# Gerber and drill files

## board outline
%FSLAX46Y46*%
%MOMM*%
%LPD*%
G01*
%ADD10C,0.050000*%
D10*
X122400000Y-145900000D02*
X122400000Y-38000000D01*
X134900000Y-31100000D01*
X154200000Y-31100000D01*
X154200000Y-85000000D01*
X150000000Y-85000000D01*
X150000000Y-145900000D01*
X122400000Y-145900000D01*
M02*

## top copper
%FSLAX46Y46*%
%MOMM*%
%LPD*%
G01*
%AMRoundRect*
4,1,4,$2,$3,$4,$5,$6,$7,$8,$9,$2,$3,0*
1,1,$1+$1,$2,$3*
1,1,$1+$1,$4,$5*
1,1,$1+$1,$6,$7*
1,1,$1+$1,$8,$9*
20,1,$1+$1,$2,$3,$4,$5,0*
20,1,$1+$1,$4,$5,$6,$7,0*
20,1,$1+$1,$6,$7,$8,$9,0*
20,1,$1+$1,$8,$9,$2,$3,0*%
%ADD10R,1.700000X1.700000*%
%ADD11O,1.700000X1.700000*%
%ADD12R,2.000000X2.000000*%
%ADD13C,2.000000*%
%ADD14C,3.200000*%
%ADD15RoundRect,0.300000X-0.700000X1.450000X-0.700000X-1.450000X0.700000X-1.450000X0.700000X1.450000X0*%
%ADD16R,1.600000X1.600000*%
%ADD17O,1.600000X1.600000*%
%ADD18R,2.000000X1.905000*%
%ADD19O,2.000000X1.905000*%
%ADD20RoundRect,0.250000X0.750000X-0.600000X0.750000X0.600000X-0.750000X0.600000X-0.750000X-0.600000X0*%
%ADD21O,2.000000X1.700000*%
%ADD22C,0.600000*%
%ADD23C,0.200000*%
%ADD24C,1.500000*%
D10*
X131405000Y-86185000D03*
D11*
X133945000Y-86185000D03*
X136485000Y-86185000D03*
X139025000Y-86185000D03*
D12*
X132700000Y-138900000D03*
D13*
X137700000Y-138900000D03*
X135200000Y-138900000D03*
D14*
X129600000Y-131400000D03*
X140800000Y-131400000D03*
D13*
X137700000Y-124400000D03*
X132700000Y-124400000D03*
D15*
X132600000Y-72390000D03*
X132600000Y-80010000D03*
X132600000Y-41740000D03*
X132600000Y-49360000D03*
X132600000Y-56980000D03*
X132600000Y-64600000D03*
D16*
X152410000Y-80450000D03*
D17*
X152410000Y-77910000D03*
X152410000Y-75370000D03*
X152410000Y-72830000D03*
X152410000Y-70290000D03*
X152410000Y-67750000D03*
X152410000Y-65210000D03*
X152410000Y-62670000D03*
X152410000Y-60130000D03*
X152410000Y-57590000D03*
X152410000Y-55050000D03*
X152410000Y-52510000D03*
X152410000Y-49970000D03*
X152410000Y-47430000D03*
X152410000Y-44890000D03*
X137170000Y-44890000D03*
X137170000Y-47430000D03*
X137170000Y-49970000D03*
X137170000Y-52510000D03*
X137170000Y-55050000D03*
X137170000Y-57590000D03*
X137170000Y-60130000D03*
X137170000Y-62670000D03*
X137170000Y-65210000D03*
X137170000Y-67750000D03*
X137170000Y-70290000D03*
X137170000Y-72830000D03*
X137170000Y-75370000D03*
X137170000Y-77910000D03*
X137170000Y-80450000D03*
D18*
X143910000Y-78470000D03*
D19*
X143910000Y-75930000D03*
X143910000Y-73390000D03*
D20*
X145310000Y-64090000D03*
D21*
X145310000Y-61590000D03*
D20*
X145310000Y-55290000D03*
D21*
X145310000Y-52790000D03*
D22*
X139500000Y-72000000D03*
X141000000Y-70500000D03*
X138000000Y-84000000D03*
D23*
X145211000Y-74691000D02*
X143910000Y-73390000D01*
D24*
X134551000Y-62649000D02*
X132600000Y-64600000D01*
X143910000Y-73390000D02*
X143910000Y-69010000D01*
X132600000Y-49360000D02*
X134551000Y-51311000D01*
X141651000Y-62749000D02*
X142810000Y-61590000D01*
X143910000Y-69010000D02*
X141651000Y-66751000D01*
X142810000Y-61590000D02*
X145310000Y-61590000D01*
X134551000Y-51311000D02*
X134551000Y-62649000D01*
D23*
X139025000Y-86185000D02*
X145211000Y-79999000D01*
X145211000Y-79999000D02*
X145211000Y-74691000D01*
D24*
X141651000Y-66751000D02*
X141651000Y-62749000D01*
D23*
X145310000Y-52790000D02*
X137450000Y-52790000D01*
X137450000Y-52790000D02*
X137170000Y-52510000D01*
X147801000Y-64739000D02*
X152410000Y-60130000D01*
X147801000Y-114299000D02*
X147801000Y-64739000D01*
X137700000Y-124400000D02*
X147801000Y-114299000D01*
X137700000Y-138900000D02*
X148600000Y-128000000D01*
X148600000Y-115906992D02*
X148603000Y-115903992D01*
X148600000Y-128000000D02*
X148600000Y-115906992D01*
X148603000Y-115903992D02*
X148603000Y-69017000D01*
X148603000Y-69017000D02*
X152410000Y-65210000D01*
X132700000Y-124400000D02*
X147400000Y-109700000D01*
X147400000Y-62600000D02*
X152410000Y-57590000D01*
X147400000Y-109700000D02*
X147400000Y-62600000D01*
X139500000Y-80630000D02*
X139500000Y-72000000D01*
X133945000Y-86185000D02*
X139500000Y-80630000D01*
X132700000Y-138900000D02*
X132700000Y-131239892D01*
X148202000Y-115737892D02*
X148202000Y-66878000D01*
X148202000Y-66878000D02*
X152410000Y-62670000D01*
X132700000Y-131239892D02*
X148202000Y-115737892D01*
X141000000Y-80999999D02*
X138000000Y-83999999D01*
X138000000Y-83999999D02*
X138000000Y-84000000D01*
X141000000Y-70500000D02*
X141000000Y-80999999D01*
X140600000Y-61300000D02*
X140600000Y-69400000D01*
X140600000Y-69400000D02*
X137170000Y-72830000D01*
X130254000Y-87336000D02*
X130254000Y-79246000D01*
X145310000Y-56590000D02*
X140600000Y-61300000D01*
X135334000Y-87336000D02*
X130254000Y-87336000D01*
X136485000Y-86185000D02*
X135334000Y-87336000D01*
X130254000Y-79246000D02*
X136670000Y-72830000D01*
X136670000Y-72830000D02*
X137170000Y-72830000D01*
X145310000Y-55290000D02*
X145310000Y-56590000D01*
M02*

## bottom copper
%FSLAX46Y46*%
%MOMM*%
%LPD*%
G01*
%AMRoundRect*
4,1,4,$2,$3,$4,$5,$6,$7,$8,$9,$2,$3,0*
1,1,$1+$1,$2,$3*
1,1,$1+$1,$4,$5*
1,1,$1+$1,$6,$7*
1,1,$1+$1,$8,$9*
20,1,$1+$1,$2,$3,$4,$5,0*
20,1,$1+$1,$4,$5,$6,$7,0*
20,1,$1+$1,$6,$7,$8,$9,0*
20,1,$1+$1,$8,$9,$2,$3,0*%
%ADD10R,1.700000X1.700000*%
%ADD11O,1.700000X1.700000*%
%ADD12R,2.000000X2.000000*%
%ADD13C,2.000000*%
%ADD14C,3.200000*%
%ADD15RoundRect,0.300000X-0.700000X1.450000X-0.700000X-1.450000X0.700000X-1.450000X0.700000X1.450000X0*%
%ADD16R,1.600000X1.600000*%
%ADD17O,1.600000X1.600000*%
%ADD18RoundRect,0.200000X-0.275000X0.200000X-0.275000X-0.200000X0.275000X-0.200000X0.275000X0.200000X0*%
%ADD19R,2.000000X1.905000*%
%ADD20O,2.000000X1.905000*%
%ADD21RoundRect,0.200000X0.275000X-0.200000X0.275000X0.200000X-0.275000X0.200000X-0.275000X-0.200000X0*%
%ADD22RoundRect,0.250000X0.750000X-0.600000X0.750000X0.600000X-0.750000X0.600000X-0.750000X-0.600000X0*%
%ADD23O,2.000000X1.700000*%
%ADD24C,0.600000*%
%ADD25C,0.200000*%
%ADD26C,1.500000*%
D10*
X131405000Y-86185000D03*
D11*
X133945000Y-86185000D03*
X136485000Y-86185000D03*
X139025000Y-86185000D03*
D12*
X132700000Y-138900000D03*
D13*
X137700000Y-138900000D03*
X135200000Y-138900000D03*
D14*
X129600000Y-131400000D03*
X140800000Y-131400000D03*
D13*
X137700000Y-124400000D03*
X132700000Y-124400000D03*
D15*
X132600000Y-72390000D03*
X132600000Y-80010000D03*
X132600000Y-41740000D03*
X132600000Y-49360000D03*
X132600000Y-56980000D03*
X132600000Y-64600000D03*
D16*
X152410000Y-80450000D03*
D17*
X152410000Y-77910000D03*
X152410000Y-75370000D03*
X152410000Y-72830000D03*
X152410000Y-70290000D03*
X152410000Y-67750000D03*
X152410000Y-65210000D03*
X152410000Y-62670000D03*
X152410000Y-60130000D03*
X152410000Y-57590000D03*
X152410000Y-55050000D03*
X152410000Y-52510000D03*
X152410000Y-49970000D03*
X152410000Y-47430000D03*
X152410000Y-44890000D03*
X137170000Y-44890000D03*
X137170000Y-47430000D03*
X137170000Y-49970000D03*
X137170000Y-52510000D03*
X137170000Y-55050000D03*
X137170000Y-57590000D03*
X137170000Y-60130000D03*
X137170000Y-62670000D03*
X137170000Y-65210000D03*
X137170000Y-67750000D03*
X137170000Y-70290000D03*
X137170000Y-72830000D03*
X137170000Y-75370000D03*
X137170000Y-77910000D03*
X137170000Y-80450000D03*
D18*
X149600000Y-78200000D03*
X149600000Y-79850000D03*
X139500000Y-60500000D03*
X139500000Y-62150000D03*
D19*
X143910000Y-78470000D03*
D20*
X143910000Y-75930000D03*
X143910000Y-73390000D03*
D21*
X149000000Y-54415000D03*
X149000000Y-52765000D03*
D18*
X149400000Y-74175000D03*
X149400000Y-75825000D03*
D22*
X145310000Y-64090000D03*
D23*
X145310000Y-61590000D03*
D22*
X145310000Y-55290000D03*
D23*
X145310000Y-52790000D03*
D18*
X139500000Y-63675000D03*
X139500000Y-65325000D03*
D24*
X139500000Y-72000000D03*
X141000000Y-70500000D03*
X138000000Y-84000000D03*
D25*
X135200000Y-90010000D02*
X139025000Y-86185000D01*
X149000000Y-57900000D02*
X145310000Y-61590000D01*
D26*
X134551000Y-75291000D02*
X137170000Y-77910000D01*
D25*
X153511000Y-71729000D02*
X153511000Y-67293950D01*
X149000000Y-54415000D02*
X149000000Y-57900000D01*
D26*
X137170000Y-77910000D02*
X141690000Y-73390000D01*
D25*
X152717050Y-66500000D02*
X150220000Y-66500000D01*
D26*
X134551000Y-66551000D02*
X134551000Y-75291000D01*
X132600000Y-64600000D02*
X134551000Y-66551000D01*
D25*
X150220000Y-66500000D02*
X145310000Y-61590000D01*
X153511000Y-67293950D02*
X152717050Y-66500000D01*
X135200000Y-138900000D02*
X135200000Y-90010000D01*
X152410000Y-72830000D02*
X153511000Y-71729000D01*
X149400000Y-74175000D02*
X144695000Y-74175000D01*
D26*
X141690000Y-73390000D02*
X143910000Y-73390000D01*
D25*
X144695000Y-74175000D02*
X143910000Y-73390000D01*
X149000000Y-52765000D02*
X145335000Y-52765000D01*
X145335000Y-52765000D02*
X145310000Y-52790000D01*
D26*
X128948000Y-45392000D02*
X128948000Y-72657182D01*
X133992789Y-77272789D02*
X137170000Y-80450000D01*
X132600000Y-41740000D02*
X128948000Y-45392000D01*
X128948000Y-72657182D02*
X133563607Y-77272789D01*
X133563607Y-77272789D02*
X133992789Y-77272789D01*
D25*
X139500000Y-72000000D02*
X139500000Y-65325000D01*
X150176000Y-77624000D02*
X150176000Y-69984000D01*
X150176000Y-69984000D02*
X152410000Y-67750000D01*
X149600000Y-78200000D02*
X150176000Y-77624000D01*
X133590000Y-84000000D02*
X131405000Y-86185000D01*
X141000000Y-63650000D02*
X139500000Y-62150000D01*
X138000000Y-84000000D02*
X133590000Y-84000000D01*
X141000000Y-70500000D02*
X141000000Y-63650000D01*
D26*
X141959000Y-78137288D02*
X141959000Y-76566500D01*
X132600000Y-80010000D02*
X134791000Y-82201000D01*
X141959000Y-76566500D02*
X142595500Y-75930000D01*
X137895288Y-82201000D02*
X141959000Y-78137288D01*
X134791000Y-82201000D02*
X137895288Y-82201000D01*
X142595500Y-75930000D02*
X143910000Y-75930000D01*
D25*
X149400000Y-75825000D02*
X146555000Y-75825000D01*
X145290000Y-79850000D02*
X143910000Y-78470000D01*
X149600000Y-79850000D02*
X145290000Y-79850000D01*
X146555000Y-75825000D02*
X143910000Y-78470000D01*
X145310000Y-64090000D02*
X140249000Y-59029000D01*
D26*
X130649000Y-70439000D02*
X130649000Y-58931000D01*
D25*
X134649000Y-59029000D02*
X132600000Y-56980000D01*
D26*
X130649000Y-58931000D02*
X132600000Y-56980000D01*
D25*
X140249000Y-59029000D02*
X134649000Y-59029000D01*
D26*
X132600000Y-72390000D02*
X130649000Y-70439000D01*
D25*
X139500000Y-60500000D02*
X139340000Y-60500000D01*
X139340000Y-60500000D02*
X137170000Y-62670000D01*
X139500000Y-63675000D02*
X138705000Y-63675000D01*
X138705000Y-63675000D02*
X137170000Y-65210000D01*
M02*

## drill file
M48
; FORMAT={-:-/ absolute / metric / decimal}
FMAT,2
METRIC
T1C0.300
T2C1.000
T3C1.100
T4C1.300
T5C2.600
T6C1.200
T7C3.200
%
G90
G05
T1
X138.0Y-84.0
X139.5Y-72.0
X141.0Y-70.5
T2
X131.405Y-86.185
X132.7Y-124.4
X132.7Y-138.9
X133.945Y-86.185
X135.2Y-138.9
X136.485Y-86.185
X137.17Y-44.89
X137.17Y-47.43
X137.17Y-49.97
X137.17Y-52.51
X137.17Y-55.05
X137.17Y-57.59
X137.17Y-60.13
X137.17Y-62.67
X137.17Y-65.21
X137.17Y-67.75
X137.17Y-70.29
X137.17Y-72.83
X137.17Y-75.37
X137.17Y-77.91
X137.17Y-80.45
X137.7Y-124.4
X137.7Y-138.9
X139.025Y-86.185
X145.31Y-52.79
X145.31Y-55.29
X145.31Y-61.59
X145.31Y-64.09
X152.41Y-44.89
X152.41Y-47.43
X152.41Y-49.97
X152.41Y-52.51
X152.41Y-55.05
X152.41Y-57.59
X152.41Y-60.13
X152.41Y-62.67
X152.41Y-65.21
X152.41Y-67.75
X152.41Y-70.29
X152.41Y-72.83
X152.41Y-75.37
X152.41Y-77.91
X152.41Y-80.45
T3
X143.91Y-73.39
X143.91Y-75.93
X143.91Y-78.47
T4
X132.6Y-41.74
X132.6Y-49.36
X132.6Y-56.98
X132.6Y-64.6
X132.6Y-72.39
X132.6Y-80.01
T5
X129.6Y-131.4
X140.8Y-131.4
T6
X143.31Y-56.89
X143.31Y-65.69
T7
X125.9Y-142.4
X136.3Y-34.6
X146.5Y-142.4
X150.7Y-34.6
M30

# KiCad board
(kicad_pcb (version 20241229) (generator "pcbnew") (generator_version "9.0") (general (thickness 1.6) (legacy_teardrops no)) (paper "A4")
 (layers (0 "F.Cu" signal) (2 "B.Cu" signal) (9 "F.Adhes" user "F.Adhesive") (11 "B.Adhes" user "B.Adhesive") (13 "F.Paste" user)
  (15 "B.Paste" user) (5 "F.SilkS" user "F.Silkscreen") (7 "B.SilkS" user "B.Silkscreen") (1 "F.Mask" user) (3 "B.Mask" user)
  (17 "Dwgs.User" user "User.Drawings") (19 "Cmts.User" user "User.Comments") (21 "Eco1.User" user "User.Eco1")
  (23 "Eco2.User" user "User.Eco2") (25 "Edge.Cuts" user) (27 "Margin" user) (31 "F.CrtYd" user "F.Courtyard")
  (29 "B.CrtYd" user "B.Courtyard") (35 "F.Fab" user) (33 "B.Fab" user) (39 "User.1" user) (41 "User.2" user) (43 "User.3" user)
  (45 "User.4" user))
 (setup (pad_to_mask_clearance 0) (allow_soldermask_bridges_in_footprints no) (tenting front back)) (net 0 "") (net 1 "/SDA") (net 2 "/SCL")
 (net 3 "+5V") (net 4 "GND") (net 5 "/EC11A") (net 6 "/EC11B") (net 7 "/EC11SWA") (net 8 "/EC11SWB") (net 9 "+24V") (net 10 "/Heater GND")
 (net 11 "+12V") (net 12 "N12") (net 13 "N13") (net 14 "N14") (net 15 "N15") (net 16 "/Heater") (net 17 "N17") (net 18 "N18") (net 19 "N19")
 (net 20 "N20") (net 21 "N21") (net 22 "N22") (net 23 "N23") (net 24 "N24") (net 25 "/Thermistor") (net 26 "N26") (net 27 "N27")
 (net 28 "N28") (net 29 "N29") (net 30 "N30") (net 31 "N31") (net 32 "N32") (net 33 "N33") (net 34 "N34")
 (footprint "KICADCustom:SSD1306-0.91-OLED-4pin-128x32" (layer "F.Cu") (at 129.215 122.685 90)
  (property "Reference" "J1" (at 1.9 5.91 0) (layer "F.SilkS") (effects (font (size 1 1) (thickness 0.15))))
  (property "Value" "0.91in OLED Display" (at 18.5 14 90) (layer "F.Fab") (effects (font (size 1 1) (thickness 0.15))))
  (pad "1" thru_hole rect (at 36.5 2.19 90) (size 1.7 1.7) (drill 1) (layers "*.Cu" "*.Mask") (remove_unused_layers no) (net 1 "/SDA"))
  (pad "2" thru_hole oval (at 36.5 4.73 90) (size 1.7 1.7) (drill 1) (layers "*.Cu" "*.Mask") (remove_unused_layers no) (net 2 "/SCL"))
  (pad "3" thru_hole oval (at 36.5 7.27 90) (size 1.7 1.7) (drill 1) (layers "*.Cu" "*.Mask") (remove_unused_layers no) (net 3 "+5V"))
  (pad "4" thru_hole oval (at 36.5 9.81 90) (size 1.7 1.7) (drill 1) (layers "*.Cu" "*.Mask") (remove_unused_layers no) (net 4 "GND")))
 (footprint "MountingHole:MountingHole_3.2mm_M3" (layer "F.Cu") (at 146.5 142.4)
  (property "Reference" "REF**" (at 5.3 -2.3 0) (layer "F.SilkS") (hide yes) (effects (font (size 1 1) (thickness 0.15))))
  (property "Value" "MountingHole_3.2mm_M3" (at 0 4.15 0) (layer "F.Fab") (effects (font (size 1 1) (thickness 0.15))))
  (pad "" np_thru_hole circle (at 0 0) (size 3.2 3.2) (drill 3.2) (layers "*.Cu" "*.Mask")))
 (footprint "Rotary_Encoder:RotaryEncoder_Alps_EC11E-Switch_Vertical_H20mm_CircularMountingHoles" (layer "F.Cu") (at 132.7 138.9 90)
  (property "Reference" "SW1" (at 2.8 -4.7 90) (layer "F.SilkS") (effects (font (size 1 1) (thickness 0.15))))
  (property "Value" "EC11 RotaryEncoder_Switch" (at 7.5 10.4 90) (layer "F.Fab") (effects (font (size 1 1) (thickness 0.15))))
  (pad "A" thru_hole rect (at 0 0 90) (size 2 2) (drill 1) (layers "*.Cu" "*.Mask") (remove_unused_layers no) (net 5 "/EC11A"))
  (pad "B" thru_hole circle (at 0 5 90) (size 2 2) (drill 1) (layers "*.Cu" "*.Mask") (remove_unused_layers no) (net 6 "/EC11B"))
  (pad "C" thru_hole circle (at 0 2.5 90) (size 2 2) (drill 1) (layers "*.Cu" "*.Mask") (remove_unused_layers no) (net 4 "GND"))
  (pad "MP" thru_hole circle (at 7.5 -3.1 90) (size 3.2 3.2) (drill 2.6) (layers "*.Cu" "*.Mask") (remove_unused_layers no))
  (pad "MP" thru_hole circle (at 7.5 8.1 90) (size 3.2 3.2) (drill 2.6) (layers "*.Cu" "*.Mask") (remove_unused_layers no))
  (pad "S1" thru_hole circle (at 14.5 5 90) (size 2 2) (drill 1) (layers "*.Cu" "*.Mask") (remove_unused_layers no) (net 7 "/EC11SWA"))
  (pad "S2" thru_hole circle (at 14.5 0 90) (size 2 2) (drill 1) (layers "*.Cu" "*.Mask") (remove_unused_layers no) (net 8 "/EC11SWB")))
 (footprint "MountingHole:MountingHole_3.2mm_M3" (layer "F.Cu") (at 136.3 34.6)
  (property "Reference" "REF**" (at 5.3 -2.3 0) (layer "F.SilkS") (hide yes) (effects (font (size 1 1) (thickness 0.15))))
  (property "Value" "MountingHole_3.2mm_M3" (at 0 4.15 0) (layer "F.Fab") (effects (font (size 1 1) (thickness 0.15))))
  (pad "" np_thru_hole circle (at 0 0) (size 3.2 3.2) (drill 3.2) (layers "*.Cu" "*.Mask")))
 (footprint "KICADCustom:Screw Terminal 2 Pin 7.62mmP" (layer "F.Cu") (at 132.6 72.39 -90)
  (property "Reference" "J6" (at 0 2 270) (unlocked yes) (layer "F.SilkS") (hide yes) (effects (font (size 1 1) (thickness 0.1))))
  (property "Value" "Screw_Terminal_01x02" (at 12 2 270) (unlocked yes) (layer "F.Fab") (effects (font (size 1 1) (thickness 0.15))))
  (pad "1" thru_hole roundrect (at 0 0 270) (size 3.5 2) (drill 1.3) (layers "*.Cu" "*.Mask") (remove_unused_layers no)
   (roundrect_rratio 0.15) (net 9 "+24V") (thermal_bridge_angle 45))
  (pad "2" thru_hole roundrect (at 7.62 0 270) (size 3.5 2) (drill 1.3) (layers "*.Cu" "*.Mask") (remove_unused_layers no)
   (roundrect_rratio 0.15) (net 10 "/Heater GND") (thermal_bridge_angle 45)))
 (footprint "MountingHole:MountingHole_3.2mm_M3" (layer "F.Cu") (at 150.7 34.6)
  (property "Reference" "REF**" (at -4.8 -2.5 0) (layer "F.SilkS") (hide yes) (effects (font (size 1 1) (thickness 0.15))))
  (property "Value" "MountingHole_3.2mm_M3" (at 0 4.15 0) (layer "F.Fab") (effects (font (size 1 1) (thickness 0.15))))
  (pad "" np_thru_hole circle (at 0 0) (size 3.2 3.2) (drill 3.2) (layers "*.Cu" "*.Mask")))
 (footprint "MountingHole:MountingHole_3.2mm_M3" (layer "F.Cu") (at 125.9 142.4)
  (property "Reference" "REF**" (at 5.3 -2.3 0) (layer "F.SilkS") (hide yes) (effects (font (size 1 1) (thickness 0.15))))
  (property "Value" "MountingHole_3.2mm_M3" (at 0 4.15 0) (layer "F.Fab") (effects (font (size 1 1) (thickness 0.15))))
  (pad "" np_thru_hole circle (at 0 0) (size 3.2 3.2) (drill 3.2) (layers "*.Cu" "*.Mask")))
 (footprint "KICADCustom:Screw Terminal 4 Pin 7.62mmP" (layer "F.Cu") (at 132.6 41.74 -90)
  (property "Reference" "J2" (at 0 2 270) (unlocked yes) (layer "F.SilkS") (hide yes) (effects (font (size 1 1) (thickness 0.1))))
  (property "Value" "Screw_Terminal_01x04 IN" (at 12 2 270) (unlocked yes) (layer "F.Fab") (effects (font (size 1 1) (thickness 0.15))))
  (pad "1" thru_hole roundrect (at 0 0 270) (size 3.5 2) (drill 1.3) (layers "*.Cu" "*.Mask") (remove_unused_layers no)
   (roundrect_rratio 0.15) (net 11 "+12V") (thermal_bridge_angle 45))
  (pad "2" thru_hole roundrect (at 7.62 0 270) (size 3.5 2) (drill 1.3) (layers "*.Cu" "*.Mask") (remove_unused_layers no)
   (roundrect_rratio 0.15) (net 4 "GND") (thermal_bridge_angle 45))
  (pad "3" thru_hole roundrect (at 15.24 0 270) (size 3.5 2) (drill 1.3) (layers "*.Cu" "*.Mask") (remove_unused_layers no)
   (roundrect_rratio 0.15) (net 9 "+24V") (thermal_bridge_angle 45))
  (pad "4" thru_hole roundrect (at 22.86 0 270) (size 3.5 2) (drill 1.3) (layers "*.Cu" "*.Mask") (remove_unused_layers no)
   (roundrect_rratio 0.15) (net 4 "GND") (thermal_bridge_angle 45)))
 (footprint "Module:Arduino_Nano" (layer "F.Cu") (at 152.41 80.45 180)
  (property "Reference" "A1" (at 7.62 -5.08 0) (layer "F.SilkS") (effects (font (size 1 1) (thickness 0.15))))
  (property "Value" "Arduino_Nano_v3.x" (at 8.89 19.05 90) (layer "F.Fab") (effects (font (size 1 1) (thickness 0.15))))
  (pad "1" thru_hole rect (at 0 0 180) (size 1.6 1.6) (drill 1) (layers "*.Cu" "*.Mask") (remove_unused_layers no) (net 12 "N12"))
  (pad "2" thru_hole oval (at 0 2.54 180) (size 1.6 1.6) (drill 1) (layers "*.Cu" "*.Mask") (remove_unused_layers no) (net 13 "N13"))
  (pad "3" thru_hole oval (at 0 5.08 180) (size 1.6 1.6) (drill 1) (layers "*.Cu" "*.Mask") (remove_unused_layers no) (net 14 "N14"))
  (pad "4" thru_hole oval (at 0 7.62 180) (size 1.6 1.6) (drill 1) (layers "*.Cu" "*.Mask") (remove_unused_layers no) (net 4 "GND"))
  (pad "5" thru_hole oval (at 0 10.16 180) (size 1.6 1.6) (drill 1) (layers "*.Cu" "*.Mask") (remove_unused_layers no) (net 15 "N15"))
  (pad "6" thru_hole oval (at 0 12.7 180) (size 1.6 1.6) (drill 1) (layers "*.Cu" "*.Mask") (remove_unused_layers no) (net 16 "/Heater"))
  (pad "7" thru_hole oval (at 0 15.24 180) (size 1.6 1.6) (drill 1) (layers "*.Cu" "*.Mask") (remove_unused_layers no) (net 6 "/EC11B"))
  (pad "8" thru_hole oval (at 0 17.78 180) (size 1.6 1.6) (drill 1) (layers "*.Cu" "*.Mask") (remove_unused_layers no) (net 5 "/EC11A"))
  (pad "9" thru_hole oval (at 0 20.32 180) (size 1.6 1.6) (drill 1) (layers "*.Cu" "*.Mask") (remove_unused_layers no) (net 7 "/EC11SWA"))
  (pad "10" thru_hole oval (at 0 22.86 180) (size 1.6 1.6) (drill 1) (layers "*.Cu" "*.Mask") (remove_unused_layers no) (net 8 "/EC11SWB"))
  (pad "11" thru_hole oval (at 0 25.4 180) (size 1.6 1.6) (drill 1) (layers "*.Cu" "*.Mask") (remove_unused_layers no) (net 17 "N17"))
  (pad "12" thru_hole oval (at 0 27.94 180) (size 1.6 1.6) (drill 1) (layers "*.Cu" "*.Mask") (remove_unused_layers no) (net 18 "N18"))
  (pad "13" thru_hole oval (at 0 30.48 180) (size 1.6 1.6) (drill 1) (layers "*.Cu" "*.Mask") (remove_unused_layers no) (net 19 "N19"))
  (pad "14" thru_hole oval (at 0 33.02 180) (size 1.6 1.6) (drill 1) (layers "*.Cu" "*.Mask") (remove_unused_layers no) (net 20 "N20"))
  (pad "15" thru_hole oval (at 0 35.56 180) (size 1.6 1.6) (drill 1) (layers "*.Cu" "*.Mask") (remove_unused_layers no) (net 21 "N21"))
  (pad "16" thru_hole oval (at 15.24 35.56 180) (size 1.6 1.6) (drill 1) (layers "*.Cu" "*.Mask") (remove_unused_layers no) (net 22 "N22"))
  (pad "17" thru_hole oval (at 15.24 33.02 180) (size 1.6 1.6) (drill 1) (layers "*.Cu" "*.Mask") (remove_unused_layers no) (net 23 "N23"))
  (pad "18" thru_hole oval (at 15.24 30.48 180) (size 1.6 1.6) (drill 1) (layers "*.Cu" "*.Mask") (remove_unused_layers no) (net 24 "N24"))
  (pad "19" thru_hole oval (at 15.24 27.94 180) (size 1.6 1.6) (drill 1) (layers "*.Cu" "*.Mask") (remove_unused_layers no)
   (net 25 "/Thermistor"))
  (pad "20" thru_hole oval (at 15.24 25.4 180) (size 1.6 1.6) (drill 1) (layers "*.Cu" "*.Mask") (remove_unused_layers no) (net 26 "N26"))
  (pad "21" thru_hole oval (at 15.24 22.86 180) (size 1.6 1.6) (drill 1) (layers "*.Cu" "*.Mask") (remove_unused_layers no) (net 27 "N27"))
  (pad "22" thru_hole oval (at 15.24 20.32 180) (size 1.6 1.6) (drill 1) (layers "*.Cu" "*.Mask") (remove_unused_layers no) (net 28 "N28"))
  (pad "23" thru_hole oval (at 15.24 17.78 180) (size 1.6 1.6) (drill 1) (layers "*.Cu" "*.Mask") (remove_unused_layers no) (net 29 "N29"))
  (pad "24" thru_hole oval (at 15.24 15.24 180) (size 1.6 1.6) (drill 1) (layers "*.Cu" "*.Mask") (remove_unused_layers no) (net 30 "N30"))
  (pad "25" thru_hole oval (at 15.24 12.7 180) (size 1.6 1.6) (drill 1) (layers "*.Cu" "*.Mask") (remove_unused_layers no) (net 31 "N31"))
  (pad "26" thru_hole oval (at 15.24 10.16 180) (size 1.6 1.6) (drill 1) (layers "*.Cu" "*.Mask") (remove_unused_layers no) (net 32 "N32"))
  (pad "27" thru_hole oval (at 15.24 7.62 180) (size 1.6 1.6) (drill 1) (layers "*.Cu" "*.Mask") (remove_unused_layers no) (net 3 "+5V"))
  (pad "28" thru_hole oval (at 15.24 5.08 180) (size 1.6 1.6) (drill 1) (layers "*.Cu" "*.Mask") (remove_unused_layers no) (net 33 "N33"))
  (pad "29" thru_hole oval (at 15.24 2.54 180) (size 1.6 1.6) (drill 1) (layers "*.Cu" "*.Mask") (remove_unused_layers no) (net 4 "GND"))
  (pad "30" thru_hole oval (at 15.24 0 180) (size 1.6 1.6) (drill 1) (layers "*.Cu" "*.Mask") (remove_unused_layers no) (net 11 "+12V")))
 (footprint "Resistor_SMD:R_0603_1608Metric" (layer "B.Cu") (at 149.6 79.025 -90)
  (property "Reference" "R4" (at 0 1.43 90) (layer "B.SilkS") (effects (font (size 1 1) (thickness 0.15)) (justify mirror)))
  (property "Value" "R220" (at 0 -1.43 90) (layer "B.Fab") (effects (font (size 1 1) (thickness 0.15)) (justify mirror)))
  (pad "1" smd roundrect (at -0.825 0 270) (size 0.8 0.95) (layers "B.Cu" "B.Mask" "B.Paste") (roundrect_rratio 0.25) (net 16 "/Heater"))
  (pad "2" smd roundrect (at 0.825 0 270) (size 0.8 0.95) (layers "B.Cu" "B.Mask" "B.Paste") (roundrect_rratio 0.25) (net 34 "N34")))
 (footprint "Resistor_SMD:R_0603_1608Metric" (layer "B.Cu") (at 139.5 61.325 -90)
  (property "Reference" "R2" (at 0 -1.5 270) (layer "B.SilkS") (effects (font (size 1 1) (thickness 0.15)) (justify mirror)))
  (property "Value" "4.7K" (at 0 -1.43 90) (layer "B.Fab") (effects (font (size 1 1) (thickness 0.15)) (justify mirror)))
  (pad "1" smd roundrect (at -0.825 0 270) (size 0.8 0.95) (layers "B.Cu" "B.Mask" "B.Paste") (roundrect_rratio 0.25) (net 29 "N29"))
  (pad "2" smd roundrect (at 0.825 0 270) (size 0.8 0.95) (layers "B.Cu" "B.Mask" "B.Paste") (roundrect_rratio 0.25) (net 1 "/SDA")))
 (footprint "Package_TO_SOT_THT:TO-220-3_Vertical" (layer "B.Cu") (at 143.91 78.47 90)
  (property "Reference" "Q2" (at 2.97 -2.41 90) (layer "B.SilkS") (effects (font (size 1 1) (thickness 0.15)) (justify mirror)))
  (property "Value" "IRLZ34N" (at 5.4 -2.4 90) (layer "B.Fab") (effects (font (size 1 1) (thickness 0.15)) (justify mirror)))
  (pad "1" thru_hole rect (at 0 0 90) (size 1.905 2) (drill 1.1) (layers "*.Cu" "*.Mask") (remove_unused_layers no) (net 34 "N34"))
  (pad "2" thru_hole oval (at 2.54 0 90) (size 1.905 2) (drill 1.1) (layers "*.Cu" "*.Mask") (remove_unused_layers no)
   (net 10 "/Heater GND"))
  (pad "3" thru_hole oval (at 5.08 0 90) (size 1.905 2) (drill 1.1) (layers "*.Cu" "*.Mask") (remove_unused_layers no) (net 4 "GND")))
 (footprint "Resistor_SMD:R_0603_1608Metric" (layer "B.Cu") (at 149 53.59 90)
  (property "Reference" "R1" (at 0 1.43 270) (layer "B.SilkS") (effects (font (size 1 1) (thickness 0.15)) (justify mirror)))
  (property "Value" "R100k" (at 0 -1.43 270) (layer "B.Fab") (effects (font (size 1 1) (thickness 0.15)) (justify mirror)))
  (pad "1" smd roundrect (at -0.825 0 90) (size 0.8 0.95) (layers "B.Cu" "B.Mask" "B.Paste") (roundrect_rratio 0.25) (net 4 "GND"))
  (pad "2" smd roundrect (at 0.825 0 90) (size 0.8 0.95) (layers "B.Cu" "B.Mask" "B.Paste") (roundrect_rratio 0.25) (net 25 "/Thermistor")))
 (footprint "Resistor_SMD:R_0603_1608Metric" (layer "B.Cu") (at 149.4 75 -90)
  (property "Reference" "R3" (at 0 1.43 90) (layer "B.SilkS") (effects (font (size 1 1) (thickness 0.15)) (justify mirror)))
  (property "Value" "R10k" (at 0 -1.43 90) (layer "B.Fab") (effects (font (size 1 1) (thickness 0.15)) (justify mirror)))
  (pad "1" smd roundrect (at -0.825 0 270) (size 0.8 0.95) (layers "B.Cu" "B.Mask" "B.Paste") (roundrect_rratio 0.25) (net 4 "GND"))
  (pad "2" smd roundrect (at 0.825 0 270) (size 0.8 0.95) (layers "B.Cu" "B.Mask" "B.Paste") (roundrect_rratio 0.25) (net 34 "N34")))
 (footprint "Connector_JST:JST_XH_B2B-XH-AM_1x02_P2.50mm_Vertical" (layer "B.Cu") (at 145.31 64.09 90)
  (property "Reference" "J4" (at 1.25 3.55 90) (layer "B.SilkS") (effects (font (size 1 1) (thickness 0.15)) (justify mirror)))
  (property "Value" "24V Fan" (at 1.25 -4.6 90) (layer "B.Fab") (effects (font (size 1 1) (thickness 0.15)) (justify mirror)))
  (pad "" np_thru_hole circle (at -1.6 -2 90) (size 1.2 1.2) (drill 1.2) (layers "*.Cu" "*.Mask"))
  (pad "1" thru_hole roundrect (at 0 0 90) (size 1.7 2) (drill 1) (layers "*.Cu" "*.Mask") (remove_unused_layers no)
   (roundrect_rratio 0.147059) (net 9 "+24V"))
  (pad "2" thru_hole oval (at 2.5 0 90) (size 1.7 2) (drill 1) (layers "*.Cu" "*.Mask") (remove_unused_layers no) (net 4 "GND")))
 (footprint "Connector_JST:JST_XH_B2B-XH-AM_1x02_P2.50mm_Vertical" (layer "B.Cu") (at 145.31 55.29 90)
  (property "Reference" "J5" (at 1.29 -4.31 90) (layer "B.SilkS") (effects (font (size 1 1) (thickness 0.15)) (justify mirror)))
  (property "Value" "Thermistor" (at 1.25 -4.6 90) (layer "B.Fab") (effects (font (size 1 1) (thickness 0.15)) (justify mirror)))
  (pad "" np_thru_hole circle (at -1.6 -2 90) (size 1.2 1.2) (drill 1.2) (layers "*.Cu" "*.Mask"))
  (pad "1" thru_hole roundrect (at 0 0 90) (size 1.7 2) (drill 1) (layers "*.Cu" "*.Mask") (remove_unused_layers no)
   (roundrect_rratio 0.147059) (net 3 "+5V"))
  (pad "2" thru_hole oval (at 2.5 0 90) (size 1.7 2) (drill 1) (layers "*.Cu" "*.Mask") (remove_unused_layers no) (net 25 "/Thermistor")))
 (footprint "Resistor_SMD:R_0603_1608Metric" (layer "B.Cu") (at 139.5 64.5 -90)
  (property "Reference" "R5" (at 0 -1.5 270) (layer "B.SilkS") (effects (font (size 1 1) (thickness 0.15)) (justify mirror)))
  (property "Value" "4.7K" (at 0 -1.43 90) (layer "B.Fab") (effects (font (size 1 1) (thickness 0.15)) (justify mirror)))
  (pad "1" smd roundrect (at -0.825 0 270) (size 0.8 0.95) (layers "B.Cu" "B.Mask" "B.Paste") (roundrect_rratio 0.25) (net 30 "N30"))
  (pad "2" smd roundrect (at 0.825 0 270) (size 0.8 0.95) (layers "B.Cu" "B.Mask" "B.Paste") (roundrect_rratio 0.25) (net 2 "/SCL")))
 (gr_poly
  (pts (xy 122.4 145.9) (xy 122.4 38) (xy 134.9 31.1) (xy 154.2 31.1) (xy 154.2 85) (xy 150 85) (xy 150 145.9))
  (stroke (width 0.05) (type solid)) (fill no) (layer "Edge.Cuts"))
 (segment (start 145.211 74.691) (end 143.91 73.39) (width 0.2) (layer "F.Cu") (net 4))
 (segment (start 134.551 62.649) (end 132.6 64.6) (width 1.5) (layer "F.Cu") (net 4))
 (segment (start 143.91 73.39) (end 143.91 69.01) (width 1.5) (layer "F.Cu") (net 4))
 (segment (start 132.6 49.36) (end 134.551 51.311) (width 1.5) (layer "F.Cu") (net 4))
 (segment (start 141.651 62.749) (end 142.81 61.59) (width 1.5) (layer "F.Cu") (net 4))
 (segment (start 143.91 69.01) (end 141.651 66.751) (width 1.5) (layer "F.Cu") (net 4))
 (segment (start 142.81 61.59) (end 145.31 61.59) (width 1.5) (layer "F.Cu") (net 4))
 (segment (start 134.551 51.311) (end 134.551 62.649) (width 1.5) (layer "F.Cu") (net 4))
 (segment (start 139.025 86.185) (end 145.211 79.999) (width 0.2) (layer "F.Cu") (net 4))
 (segment (start 145.211 79.999) (end 145.211 74.691) (width 0.2) (layer "F.Cu") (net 4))
 (segment (start 141.651 66.751) (end 141.651 62.749) (width 1.5) (layer "F.Cu") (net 4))
 (segment (start 135.2 90.01) (end 139.025 86.185) (width 0.2) (layer "B.Cu") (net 4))
 (segment (start 149 57.9) (end 145.31 61.59) (width 0.2) (layer "B.Cu") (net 4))
 (segment (start 134.551 75.291) (end 137.17 77.91) (width 1.5) (layer "B.Cu") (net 4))
 (segment (start 153.511 71.729) (end 153.511 67.29395) (width 0.2) (layer "B.Cu") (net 4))
 (segment (start 149 54.415) (end 149 57.9) (width 0.2) (layer "B.Cu") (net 4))
 (segment (start 137.17 77.91) (end 141.69 73.39) (width 1.5) (layer "B.Cu") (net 4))
 (segment (start 152.71705 66.5) (end 150.22 66.5) (width 0.2) (layer "B.Cu") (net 4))
 (segment (start 134.551 66.551) (end 134.551 75.291) (width 1.5) (layer "B.Cu") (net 4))
 (segment (start 132.6 64.6) (end 134.551 66.551) (width 1.5) (layer "B.Cu") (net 4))
 (segment (start 150.22 66.5) (end 145.31 61.59) (width 0.2) (layer "B.Cu") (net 4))
 (segment (start 153.511 67.29395) (end 152.71705 66.5) (width 0.2) (layer "B.Cu") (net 4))
 (segment (start 135.2 138.9) (end 135.2 90.01) (width 0.2) (layer "B.Cu") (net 4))
 (segment (start 152.41 72.83) (end 153.511 71.729) (width 0.2) (layer "B.Cu") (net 4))
 (segment (start 149.4 74.175) (end 144.695 74.175) (width 0.2) (layer "B.Cu") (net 4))
 (segment (start 141.69 73.39) (end 143.91 73.39) (width 1.5) (layer "B.Cu") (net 4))
 (segment (start 144.695 74.175) (end 143.91 73.39) (width 0.2) (layer "B.Cu") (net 4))
 (segment (start 145.31 52.79) (end 137.45 52.79) (width 0.2) (layer "F.Cu") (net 25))
 (segment (start 137.45 52.79) (end 137.17 52.51) (width 0.2) (layer "F.Cu") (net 25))
 (segment (start 149 52.765) (end 145.335 52.765) (width 0.2) (layer "B.Cu") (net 25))
 (segment (start 145.335 52.765) (end 145.31 52.79) (width 0.2) (layer "B.Cu") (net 25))
 (segment (start 147.801 64.739) (end 152.41 60.13) (width 0.2) (layer "F.Cu") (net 7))
 (segment (start 147.801 114.299) (end 147.801 64.739) (width 0.2) (layer "F.Cu") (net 7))
 (segment (start 137.7 124.4) (end 147.801 114.299) (width 0.2) (layer "F.Cu") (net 7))
 (segment (start 137.7 138.9) (end 148.6 128) (width 0.2) (layer "F.Cu") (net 6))
 (segment (start 148.6 115.906992) (end 148.603 115.903992) (width 0.2) (layer "F.Cu") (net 6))
 (segment (start 148.6 128) (end 148.6 115.906992) (width 0.2) (layer "F.Cu") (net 6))
 (segment (start 148.603 115.903992) (end 148.603 69.017) (width 0.2) (layer "F.Cu") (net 6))
 (segment (start 148.603 69.017) (end 152.41 65.21) (width 0.2) (layer "F.Cu") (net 6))
 (segment (start 132.7 124.4) (end 147.4 109.7) (width 0.2) (layer "F.Cu") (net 8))
 (segment (start 147.4 62.6) (end 152.41 57.59) (width 0.2) (layer "F.Cu") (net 8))
 (segment (start 147.4 109.7) (end 147.4 62.6) (width 0.2) (layer "F.Cu") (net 8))
 (segment (start 128.948 45.392) (end 128.948 72.657182) (width 1.5) (layer "B.Cu") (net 11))
 (segment (start 133.992789 77.272789) (end 137.17 80.45) (width 1.5) (layer "B.Cu") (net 11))
 (segment (start 132.6 41.74) (end 128.948 45.392) (width 1.5) (layer "B.Cu") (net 11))
 (segment (start 128.948 72.657182) (end 133.563607 77.272789) (width 1.5) (layer "B.Cu") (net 11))
 (segment (start 133.563607 77.272789) (end 133.992789 77.272789) (width 1.5) (layer "B.Cu") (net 11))
 (segment (start 139.5 80.63) (end 139.5 72) (width 0.2) (layer "F.Cu") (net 2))
 (segment (start 133.945 86.185) (end 139.5 80.63) (width 0.2) (layer "F.Cu") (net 2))
 (via (at 139.5 72) (size 0.6) (drill 0.3) (layers "F.Cu" "B.Cu") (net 2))
 (segment (start 139.5 72) (end 139.5 65.325) (width 0.2) (layer "B.Cu") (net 2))
 (segment (start 132.7 138.9) (end 132.7 131.239892) (width 0.2) (layer "F.Cu") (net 5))
 (segment (start 148.202 115.737892) (end 148.202 66.878) (width 0.2) (layer "F.Cu") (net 5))
 (segment (start 148.202 66.878) (end 152.41 62.67) (width 0.2) (layer "F.Cu") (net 5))
 (segment (start 132.7 131.239892) (end 148.202 115.737892) (width 0.2) (layer "F.Cu") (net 5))
 (segment (start 150.176 77.624) (end 150.176 69.984) (width 0.2) (layer "B.Cu") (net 16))
 (segment (start 150.176 69.984) (end 152.41 67.75) (width 0.2) (layer "B.Cu") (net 16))
 (segment (start 149.6 78.2) (end 150.176 77.624) (width 0.2) (layer "B.Cu") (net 16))
 (segment (start 141 80.999999) (end 138 83.999999) (width 0.2) (layer "F.Cu") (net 1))
 (segment (start 138 83.999999) (end 138 84) (width 0.2) (layer "F.Cu") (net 1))
 (segment (start 141 70.5) (end 141 80.999999) (width 0.2) (layer "F.Cu") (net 1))
 (via (at 141 70.5) (size 0.6) (drill 0.3) (layers "F.Cu" "B.Cu") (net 1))
 (via (at 138 84) (size 0.6) (drill 0.3) (layers "F.Cu" "B.Cu") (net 1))
 (segment (start 133.59 84) (end 131.405 86.185) (width 0.2) (layer "B.Cu") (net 1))
 (segment (start 141 63.65) (end 139.5 62.15) (width 0.2) (layer "B.Cu") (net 1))
 (segment (start 138 84) (end 133.59 84) (width 0.2) (layer "B.Cu") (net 1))
 (segment (start 141 70.5) (end 141 63.65) (width 0.2) (layer "B.Cu") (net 1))
 (segment (start 140.6 61.3) (end 140.6 69.4) (width 0.2) (layer "F.Cu") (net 3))
 (segment (start 140.6 69.4) (end 137.17 72.83) (width 0.2) (layer "F.Cu") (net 3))
 (segment (start 130.254 87.336) (end 130.254 79.246) (width 0.2) (layer "F.Cu") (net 3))
 (segment (start 145.31 56.59) (end 140.6 61.3) (width 0.2) (layer "F.Cu") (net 3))
 (segment (start 135.334 87.336) (end 130.254 87.336) (width 0.2) (layer "F.Cu") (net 3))
 (segment (start 136.485 86.185) (end 135.334 87.336) (width 0.2) (layer "F.Cu") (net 3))
 (segment (start 130.254 79.246) (end 136.67 72.83) (width 0.2) (layer "F.Cu") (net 3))
 (segment (start 136.67 72.83) (end 137.17 72.83) (width 0.2) (layer "F.Cu") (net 3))
 (segment (start 145.31 55.29) (end 145.31 56.59) (width 0.2) (layer "F.Cu") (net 3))
 (segment (start 141.959 78.137288) (end 141.959 76.5665) (width 1.5) (layer "B.Cu") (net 10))
 (segment (start 132.6 80.01) (end 134.791 82.201) (width 1.5) (layer "B.Cu") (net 10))
 (segment (start 141.959 76.5665) (end 142.5955 75.93) (width 1.5) (layer "B.Cu") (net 10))
 (segment (start 137.895288 82.201) (end 141.959 78.137288) (width 1.5) (layer "B.Cu") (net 10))
 (segment (start 134.791 82.201) (end 137.895288 82.201) (width 1.5) (layer "B.Cu") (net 10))
 (segment (start 142.5955 75.93) (end 143.91 75.93) (width 1.5) (layer "B.Cu") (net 10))
 (segment (start 149.4 75.825) (end 146.555 75.825) (width 0.2) (layer "B.Cu") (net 34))
 (segment (start 145.29 79.85) (end 143.91 78.47) (width 0.2) (layer "B.Cu") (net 34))
 (segment (start 149.6 79.85) (end 145.29 79.85) (width 0.2) (layer "B.Cu") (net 34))
 (segment (start 146.555 75.825) (end 143.91 78.47) (width 0.2) (layer "B.Cu") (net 34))
 (segment (start 145.31 64.09) (end 140.249 59.029) (width 0.2) (layer "B.Cu") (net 9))
 (segment (start 130.649 70.439) (end 130.649 58.931) (width 1.5) (layer "B.Cu") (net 9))
 (segment (start 134.649 59.029) (end 132.6 56.98) (width 0.2) (layer "B.Cu") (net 9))
 (segment (start 130.649 58.931) (end 132.6 56.98) (width 1.5) (layer "B.Cu") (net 9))
 (segment (start 140.249 59.029) (end 134.649 59.029) (width 0.2) (layer "B.Cu") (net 9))
 (segment (start 132.6 72.39) (end 130.649 70.439) (width 1.5) (layer "B.Cu") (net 9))
 (segment (start 139.5 60.5) (end 139.34 60.5) (width 0.2) (layer "B.Cu") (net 29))
 (segment (start 139.34 60.5) (end 137.17 62.67) (width 0.2) (layer "B.Cu") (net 29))
 (segment (start 139.5 63.675) (end 138.705 63.675) (width 0.2) (layer "B.Cu") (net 30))
 (segment (start 138.705 63.675) (end 137.17 65.21) (width 0.2) (layer "B.Cu") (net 30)))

